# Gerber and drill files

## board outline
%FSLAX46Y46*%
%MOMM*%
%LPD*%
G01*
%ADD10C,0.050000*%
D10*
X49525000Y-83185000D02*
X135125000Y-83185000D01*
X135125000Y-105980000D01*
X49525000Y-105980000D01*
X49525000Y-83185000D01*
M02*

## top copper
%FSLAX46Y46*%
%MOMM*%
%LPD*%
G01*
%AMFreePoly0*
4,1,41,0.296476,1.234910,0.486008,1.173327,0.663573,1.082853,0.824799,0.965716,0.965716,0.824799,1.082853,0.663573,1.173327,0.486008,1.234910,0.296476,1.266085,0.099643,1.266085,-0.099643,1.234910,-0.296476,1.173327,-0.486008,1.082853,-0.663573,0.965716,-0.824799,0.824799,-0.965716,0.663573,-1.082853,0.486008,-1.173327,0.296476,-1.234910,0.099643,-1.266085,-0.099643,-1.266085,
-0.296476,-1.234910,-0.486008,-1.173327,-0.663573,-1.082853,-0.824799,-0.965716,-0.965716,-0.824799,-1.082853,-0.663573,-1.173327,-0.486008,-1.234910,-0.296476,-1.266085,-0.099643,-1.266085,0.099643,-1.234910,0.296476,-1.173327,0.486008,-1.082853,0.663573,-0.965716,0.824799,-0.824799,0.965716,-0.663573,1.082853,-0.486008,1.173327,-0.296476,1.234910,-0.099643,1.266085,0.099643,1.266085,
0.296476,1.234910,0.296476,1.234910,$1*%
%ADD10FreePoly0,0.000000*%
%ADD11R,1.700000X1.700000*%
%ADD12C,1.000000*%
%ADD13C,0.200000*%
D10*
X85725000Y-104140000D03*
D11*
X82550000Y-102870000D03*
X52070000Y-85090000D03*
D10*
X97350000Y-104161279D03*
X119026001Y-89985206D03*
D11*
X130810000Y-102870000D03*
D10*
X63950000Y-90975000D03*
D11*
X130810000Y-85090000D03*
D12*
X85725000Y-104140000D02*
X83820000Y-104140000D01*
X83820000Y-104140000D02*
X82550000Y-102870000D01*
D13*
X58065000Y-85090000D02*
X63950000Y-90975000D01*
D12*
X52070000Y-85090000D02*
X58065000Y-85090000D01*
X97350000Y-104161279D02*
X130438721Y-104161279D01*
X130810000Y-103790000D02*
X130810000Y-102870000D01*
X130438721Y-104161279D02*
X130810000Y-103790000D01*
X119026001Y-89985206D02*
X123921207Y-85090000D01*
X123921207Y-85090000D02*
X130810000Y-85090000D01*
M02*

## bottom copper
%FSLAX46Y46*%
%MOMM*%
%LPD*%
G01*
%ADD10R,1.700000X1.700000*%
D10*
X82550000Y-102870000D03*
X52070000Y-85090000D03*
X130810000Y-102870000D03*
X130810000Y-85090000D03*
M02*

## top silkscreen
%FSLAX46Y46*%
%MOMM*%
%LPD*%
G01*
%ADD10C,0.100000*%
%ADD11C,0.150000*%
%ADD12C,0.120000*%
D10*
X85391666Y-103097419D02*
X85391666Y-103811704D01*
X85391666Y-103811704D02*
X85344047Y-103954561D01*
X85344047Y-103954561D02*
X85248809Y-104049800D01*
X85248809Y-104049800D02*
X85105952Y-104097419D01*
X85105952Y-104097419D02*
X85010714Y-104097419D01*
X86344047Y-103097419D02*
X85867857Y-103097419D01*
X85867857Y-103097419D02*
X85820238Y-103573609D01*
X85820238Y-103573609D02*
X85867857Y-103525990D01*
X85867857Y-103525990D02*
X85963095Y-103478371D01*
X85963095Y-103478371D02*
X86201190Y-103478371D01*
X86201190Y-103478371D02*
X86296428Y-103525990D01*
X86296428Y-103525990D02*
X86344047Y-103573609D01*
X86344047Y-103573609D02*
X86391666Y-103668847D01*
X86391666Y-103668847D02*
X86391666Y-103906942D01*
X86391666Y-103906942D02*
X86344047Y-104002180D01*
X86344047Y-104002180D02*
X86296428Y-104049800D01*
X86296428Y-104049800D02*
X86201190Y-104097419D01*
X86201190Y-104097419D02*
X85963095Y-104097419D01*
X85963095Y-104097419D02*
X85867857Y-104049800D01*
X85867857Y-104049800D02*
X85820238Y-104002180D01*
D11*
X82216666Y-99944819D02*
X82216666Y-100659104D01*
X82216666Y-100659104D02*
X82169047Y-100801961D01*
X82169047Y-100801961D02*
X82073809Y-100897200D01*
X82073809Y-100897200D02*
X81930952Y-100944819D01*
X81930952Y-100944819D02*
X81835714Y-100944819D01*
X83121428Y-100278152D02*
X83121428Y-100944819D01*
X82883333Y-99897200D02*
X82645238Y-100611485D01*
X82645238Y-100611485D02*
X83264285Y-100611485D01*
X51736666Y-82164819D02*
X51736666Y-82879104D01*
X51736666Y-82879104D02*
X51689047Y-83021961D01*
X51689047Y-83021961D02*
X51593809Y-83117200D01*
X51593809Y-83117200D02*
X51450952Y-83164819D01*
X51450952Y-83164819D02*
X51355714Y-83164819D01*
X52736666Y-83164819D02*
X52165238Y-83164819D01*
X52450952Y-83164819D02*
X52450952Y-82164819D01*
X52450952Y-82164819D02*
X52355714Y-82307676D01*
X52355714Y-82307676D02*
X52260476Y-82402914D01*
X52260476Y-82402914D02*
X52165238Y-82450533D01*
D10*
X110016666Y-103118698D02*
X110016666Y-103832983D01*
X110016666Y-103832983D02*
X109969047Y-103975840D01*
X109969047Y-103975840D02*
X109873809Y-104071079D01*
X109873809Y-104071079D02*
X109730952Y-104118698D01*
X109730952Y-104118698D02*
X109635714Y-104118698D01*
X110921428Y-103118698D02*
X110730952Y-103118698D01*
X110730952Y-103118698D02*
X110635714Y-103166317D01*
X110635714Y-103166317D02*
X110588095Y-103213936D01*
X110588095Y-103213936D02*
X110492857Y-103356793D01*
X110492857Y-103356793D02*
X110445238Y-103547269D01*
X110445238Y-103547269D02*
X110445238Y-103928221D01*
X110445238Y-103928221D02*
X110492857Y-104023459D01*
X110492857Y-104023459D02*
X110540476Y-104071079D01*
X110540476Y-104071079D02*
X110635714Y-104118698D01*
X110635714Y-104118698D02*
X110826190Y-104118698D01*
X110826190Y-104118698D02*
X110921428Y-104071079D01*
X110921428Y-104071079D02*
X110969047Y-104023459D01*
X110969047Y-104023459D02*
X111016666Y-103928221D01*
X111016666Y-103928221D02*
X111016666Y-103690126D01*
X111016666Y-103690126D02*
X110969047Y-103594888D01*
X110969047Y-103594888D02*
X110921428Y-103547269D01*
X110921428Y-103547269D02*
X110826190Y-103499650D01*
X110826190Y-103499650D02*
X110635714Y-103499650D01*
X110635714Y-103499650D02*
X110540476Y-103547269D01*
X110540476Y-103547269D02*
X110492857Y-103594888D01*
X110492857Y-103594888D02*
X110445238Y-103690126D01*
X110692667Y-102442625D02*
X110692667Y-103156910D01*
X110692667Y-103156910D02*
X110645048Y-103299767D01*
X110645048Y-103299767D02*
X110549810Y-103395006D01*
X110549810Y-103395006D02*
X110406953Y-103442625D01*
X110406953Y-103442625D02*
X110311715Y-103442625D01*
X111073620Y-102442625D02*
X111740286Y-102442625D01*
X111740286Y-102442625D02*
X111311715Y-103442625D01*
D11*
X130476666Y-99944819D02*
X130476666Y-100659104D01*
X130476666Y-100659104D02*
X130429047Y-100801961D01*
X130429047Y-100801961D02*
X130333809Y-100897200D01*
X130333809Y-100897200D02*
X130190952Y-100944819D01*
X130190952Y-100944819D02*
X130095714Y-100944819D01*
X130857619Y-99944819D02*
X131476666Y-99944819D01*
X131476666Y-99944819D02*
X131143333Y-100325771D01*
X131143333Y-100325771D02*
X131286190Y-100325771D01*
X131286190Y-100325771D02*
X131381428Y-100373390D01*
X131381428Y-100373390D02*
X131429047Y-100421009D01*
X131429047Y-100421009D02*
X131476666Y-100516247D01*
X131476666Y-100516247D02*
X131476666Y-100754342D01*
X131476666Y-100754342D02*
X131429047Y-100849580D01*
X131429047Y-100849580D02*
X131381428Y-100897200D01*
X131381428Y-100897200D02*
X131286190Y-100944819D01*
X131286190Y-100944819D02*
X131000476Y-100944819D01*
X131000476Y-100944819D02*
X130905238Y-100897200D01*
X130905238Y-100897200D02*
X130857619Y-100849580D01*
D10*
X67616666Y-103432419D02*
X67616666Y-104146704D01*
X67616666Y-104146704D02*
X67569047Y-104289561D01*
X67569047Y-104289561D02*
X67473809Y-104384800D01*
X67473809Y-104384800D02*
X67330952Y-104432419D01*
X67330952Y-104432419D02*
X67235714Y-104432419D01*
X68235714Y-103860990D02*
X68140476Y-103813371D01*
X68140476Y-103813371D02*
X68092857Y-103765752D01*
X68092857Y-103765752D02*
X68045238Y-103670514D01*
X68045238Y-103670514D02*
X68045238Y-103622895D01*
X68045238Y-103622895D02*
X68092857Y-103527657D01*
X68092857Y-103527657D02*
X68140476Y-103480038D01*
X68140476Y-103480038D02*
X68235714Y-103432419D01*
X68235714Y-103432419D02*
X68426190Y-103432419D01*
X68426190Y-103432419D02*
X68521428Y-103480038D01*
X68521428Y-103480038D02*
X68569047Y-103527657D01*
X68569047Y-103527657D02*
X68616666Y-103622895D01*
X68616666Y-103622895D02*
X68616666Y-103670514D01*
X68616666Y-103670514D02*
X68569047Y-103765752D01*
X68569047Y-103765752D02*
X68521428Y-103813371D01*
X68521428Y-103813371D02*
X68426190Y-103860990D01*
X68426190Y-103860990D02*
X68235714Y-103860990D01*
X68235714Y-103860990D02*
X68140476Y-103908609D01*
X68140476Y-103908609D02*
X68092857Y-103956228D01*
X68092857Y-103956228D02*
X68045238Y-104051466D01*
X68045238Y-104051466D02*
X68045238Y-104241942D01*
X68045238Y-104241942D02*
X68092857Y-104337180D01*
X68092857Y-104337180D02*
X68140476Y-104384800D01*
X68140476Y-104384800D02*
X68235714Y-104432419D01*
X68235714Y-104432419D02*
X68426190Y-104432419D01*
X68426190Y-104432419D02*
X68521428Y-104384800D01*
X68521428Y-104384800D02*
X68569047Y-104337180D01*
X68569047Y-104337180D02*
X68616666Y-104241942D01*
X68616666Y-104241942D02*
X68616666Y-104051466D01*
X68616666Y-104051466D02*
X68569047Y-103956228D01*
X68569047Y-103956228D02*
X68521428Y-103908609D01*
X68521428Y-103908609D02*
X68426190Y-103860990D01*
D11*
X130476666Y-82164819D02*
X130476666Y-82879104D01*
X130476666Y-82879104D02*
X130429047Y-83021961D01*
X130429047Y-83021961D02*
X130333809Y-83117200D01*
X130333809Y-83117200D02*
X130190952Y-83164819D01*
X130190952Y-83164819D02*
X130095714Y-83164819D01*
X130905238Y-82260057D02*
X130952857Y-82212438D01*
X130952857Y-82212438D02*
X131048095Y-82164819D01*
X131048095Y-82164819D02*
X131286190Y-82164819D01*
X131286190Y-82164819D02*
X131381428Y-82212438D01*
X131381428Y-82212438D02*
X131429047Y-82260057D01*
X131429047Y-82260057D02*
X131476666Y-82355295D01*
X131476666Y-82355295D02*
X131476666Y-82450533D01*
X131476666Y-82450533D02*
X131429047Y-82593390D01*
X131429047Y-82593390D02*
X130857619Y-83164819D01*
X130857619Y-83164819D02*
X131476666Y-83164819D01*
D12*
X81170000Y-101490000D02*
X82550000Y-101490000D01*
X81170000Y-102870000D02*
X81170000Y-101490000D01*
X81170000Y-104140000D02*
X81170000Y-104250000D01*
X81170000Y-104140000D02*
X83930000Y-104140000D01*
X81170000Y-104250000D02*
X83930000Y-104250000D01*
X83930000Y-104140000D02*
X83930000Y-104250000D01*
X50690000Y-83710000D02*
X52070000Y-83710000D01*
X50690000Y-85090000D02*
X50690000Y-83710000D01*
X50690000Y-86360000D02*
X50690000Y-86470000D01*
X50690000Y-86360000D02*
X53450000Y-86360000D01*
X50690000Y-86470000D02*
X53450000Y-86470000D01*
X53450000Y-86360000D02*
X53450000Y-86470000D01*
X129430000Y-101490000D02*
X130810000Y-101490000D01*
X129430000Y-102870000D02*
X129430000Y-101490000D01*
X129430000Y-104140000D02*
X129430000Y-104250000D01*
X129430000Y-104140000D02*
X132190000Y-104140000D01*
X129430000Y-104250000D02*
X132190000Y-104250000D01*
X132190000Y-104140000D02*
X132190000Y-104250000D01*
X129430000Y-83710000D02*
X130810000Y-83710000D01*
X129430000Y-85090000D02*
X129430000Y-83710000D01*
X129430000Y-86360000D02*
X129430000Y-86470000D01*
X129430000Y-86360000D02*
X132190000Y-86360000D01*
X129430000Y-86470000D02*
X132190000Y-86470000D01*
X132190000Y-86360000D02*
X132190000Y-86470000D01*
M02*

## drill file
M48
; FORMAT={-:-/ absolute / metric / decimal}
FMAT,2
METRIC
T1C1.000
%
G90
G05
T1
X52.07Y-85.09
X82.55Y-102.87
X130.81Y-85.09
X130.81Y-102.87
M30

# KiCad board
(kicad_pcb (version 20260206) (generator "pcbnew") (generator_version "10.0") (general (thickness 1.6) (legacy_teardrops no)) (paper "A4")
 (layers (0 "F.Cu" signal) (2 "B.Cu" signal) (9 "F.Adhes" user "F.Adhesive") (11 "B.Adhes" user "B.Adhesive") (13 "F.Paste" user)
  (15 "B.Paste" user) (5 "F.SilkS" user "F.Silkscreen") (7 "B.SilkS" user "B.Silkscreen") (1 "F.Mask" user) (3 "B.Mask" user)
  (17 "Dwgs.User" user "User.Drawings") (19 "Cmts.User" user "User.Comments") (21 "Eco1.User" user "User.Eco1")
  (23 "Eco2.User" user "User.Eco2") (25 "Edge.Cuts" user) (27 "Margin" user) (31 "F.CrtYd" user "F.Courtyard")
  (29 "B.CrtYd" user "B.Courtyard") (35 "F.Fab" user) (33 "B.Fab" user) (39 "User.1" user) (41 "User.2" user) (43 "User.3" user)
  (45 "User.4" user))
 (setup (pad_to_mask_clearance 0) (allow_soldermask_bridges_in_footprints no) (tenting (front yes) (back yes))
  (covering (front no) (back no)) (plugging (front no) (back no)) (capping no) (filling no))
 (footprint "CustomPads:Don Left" (layer "F.Cu") (at 85.725 104.14)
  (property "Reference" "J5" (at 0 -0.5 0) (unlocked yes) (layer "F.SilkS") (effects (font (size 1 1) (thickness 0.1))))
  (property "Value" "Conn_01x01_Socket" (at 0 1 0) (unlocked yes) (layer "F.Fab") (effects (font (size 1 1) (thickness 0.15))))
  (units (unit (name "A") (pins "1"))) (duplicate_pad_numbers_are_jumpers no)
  (pad "1" smd custom (at 0 0) (size 2.54 2.54) (layers "F.Cu" "F.Mask" "F.Paste") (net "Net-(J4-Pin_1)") (thermal_bridge_angle 90)
   (options (clearance outline) (anchor circle)) (primitives)))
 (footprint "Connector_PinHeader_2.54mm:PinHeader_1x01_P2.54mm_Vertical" (layer "F.Cu") (at 82.55 102.87)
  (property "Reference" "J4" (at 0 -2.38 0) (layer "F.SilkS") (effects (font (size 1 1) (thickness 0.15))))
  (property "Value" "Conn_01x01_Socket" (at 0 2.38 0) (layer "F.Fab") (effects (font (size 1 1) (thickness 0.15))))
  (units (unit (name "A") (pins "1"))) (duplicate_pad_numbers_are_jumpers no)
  (fp_line (start -1.38 -1.38) (end 0 -1.38) (stroke (width 0.12) (type solid)) (layer "F.SilkS"))
  (fp_line (start -1.38 0) (end -1.38 -1.38) (stroke (width 0.12) (type solid)) (layer "F.SilkS"))
  (fp_line (start -1.38 1.27) (end -1.38 1.38) (stroke (width 0.12) (type solid)) (layer "F.SilkS"))
  (fp_line (start -1.38 1.27) (end 1.38 1.27) (stroke (width 0.12) (type solid)) (layer "F.SilkS"))
  (fp_line (start -1.38 1.38) (end 1.38 1.38) (stroke (width 0.12) (type solid)) (layer "F.SilkS"))
  (fp_line (start 1.38 1.27) (end 1.38 1.38) (stroke (width 0.12) (type solid)) (layer "F.SilkS"))
  (pad "1" thru_hole rect (at 0 0) (size 1.7 1.7) (drill 1) (layers "*.Cu" "*.Mask") (remove_unused_layers no) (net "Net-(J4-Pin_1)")))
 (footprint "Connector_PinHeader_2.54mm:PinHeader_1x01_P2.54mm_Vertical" (layer "F.Cu") (at 52.07 85.09)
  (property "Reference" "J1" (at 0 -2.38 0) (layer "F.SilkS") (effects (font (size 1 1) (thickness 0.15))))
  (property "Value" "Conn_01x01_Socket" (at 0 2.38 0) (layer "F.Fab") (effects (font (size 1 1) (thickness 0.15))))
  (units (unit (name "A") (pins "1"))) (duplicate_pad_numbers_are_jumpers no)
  (fp_line (start -1.38 -1.38) (end 0 -1.38) (stroke (width 0.12) (type solid)) (layer "F.SilkS"))
  (fp_line (start -1.38 0) (end -1.38 -1.38) (stroke (width 0.12) (type solid)) (layer "F.SilkS"))
  (fp_line (start -1.38 1.27) (end -1.38 1.38) (stroke (width 0.12) (type solid)) (layer "F.SilkS"))
  (fp_line (start -1.38 1.27) (end 1.38 1.27) (stroke (width 0.12) (type solid)) (layer "F.SilkS"))
  (fp_line (start -1.38 1.38) (end 1.38 1.38) (stroke (width 0.12) (type solid)) (layer "F.SilkS"))
  (fp_line (start 1.38 1.27) (end 1.38 1.38) (stroke (width 0.12) (type solid)) (layer "F.SilkS"))
  (pad "1" thru_hole rect (at 0 0) (size 1.7 1.7) (drill 1) (layers "*.Cu" "*.Mask") (remove_unused_layers no) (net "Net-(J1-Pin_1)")))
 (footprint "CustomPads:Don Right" (layer "F.Cu") (at 110.35 104.161279)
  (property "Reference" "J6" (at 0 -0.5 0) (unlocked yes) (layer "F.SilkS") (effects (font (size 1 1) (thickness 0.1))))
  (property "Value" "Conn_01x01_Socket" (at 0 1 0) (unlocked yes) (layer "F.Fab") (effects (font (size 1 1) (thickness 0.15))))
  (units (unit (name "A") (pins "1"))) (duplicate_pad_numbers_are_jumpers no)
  (pad "1" smd custom (at -13 0) (size 2.54 2.54) (layers "F.Cu" "F.Mask" "F.Paste") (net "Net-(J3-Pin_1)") (thermal_bridge_angle 90)
   (options (clearance outline) (anchor circle)) (primitives)))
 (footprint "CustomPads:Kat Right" (layer "F.Cu") (at 111.026001 103.485206)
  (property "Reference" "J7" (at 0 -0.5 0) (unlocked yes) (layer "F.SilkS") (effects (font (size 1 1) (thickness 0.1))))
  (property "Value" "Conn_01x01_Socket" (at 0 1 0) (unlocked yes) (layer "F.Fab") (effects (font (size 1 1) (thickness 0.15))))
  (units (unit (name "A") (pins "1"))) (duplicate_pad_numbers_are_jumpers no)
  (pad "1" smd custom (at 8 -13.5) (size 2.54 2.54) (layers "F.Cu" "F.Mask" "F.Paste") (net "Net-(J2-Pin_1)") (thermal_bridge_angle 90)
   (options (clearance outline) (anchor circle)) (primitives)))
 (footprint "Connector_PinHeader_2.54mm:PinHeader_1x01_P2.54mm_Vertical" (layer "F.Cu") (at 130.81 102.87)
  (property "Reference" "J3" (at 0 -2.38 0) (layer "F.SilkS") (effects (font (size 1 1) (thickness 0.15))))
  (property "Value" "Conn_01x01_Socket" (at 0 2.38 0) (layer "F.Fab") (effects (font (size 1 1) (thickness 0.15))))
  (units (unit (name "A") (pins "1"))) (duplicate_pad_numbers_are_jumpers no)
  (fp_line (start -1.38 -1.38) (end 0 -1.38) (stroke (width 0.12) (type solid)) (layer "F.SilkS"))
  (fp_line (start -1.38 0) (end -1.38 -1.38) (stroke (width 0.12) (type solid)) (layer "F.SilkS"))
  (fp_line (start -1.38 1.27) (end -1.38 1.38) (stroke (width 0.12) (type solid)) (layer "F.SilkS"))
  (fp_line (start -1.38 1.27) (end 1.38 1.27) (stroke (width 0.12) (type solid)) (layer "F.SilkS"))
  (fp_line (start -1.38 1.38) (end 1.38 1.38) (stroke (width 0.12) (type solid)) (layer "F.SilkS"))
  (fp_line (start 1.38 1.27) (end 1.38 1.38) (stroke (width 0.12) (type solid)) (layer "F.SilkS"))
  (pad "1" thru_hole rect (at 0 0) (size 1.7 1.7) (drill 1) (layers "*.Cu" "*.Mask") (remove_unused_layers no) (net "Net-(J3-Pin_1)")))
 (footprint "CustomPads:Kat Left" (layer "F.Cu") (at 67.95 104.475)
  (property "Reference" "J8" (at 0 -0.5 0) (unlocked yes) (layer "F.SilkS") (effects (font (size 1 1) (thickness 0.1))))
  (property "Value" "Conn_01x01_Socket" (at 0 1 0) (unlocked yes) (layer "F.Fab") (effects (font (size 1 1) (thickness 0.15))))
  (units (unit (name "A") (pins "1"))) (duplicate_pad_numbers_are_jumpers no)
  (pad "1" smd custom (at -4 -13.5) (size 2.54 2.54) (layers "F.Cu" "F.Mask" "F.Paste") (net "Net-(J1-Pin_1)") (thermal_bridge_angle 90)
   (options (clearance outline) (anchor circle)) (primitives)))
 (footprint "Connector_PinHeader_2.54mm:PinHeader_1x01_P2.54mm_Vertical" (layer "F.Cu") (at 130.81 85.09)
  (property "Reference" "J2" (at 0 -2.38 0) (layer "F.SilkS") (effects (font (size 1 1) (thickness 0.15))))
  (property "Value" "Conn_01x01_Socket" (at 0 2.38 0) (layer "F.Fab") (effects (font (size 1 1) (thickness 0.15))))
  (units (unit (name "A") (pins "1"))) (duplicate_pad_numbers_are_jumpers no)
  (fp_line (start -1.38 -1.38) (end 0 -1.38) (stroke (width 0.12) (type solid)) (layer "F.SilkS"))
  (fp_line (start -1.38 0) (end -1.38 -1.38) (stroke (width 0.12) (type solid)) (layer "F.SilkS"))
  (fp_line (start -1.38 1.27) (end -1.38 1.38) (stroke (width 0.12) (type solid)) (layer "F.SilkS"))
  (fp_line (start -1.38 1.27) (end 1.38 1.27) (stroke (width 0.12) (type solid)) (layer "F.SilkS"))
  (fp_line (start -1.38 1.38) (end 1.38 1.38) (stroke (width 0.12) (type solid)) (layer "F.SilkS"))
  (fp_line (start 1.38 1.27) (end 1.38 1.38) (stroke (width 0.12) (type solid)) (layer "F.SilkS"))
  (pad "1" thru_hole rect (at 0 0) (size 1.7 1.7) (drill 1) (layers "*.Cu" "*.Mask") (remove_unused_layers no) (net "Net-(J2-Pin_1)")))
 (gr_rect (start 49.525 83.185) (end 135.125 105.98) (stroke (width 0.05) (type default)) (fill no) (layer "Edge.Cuts"))
 (segment (start 85.725 104.14) (end 83.82 104.14) (width 1) (layer "F.Cu") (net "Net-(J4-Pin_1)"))
 (segment (start 83.82 104.14) (end 82.55 102.87) (width 1) (layer "F.Cu") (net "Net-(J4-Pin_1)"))
 (segment (start 58.065 85.09) (end 63.95 90.975) (width 0.2) (layer "F.Cu") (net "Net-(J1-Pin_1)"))
 (segment (start 52.07 85.09) (end 58.065 85.09) (width 1) (layer "F.Cu") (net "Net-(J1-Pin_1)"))
 (segment (start 97.35 104.161279) (end 130.438721 104.161279) (width 1) (layer "F.Cu") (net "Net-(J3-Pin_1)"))
 (segment (start 130.81 103.79) (end 130.81 102.87) (width 1) (layer "F.Cu") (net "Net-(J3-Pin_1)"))
 (segment (start 130.438721 104.161279) (end 130.81 103.79) (width 1) (layer "F.Cu") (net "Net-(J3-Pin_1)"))
 (segment (start 119.026001 89.985206) (end 123.921207 85.09) (width 1) (layer "F.Cu") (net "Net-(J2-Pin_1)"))
 (segment (start 123.921207 85.09) (end 130.81 85.09) (width 1) (layer "F.Cu") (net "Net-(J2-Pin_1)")))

